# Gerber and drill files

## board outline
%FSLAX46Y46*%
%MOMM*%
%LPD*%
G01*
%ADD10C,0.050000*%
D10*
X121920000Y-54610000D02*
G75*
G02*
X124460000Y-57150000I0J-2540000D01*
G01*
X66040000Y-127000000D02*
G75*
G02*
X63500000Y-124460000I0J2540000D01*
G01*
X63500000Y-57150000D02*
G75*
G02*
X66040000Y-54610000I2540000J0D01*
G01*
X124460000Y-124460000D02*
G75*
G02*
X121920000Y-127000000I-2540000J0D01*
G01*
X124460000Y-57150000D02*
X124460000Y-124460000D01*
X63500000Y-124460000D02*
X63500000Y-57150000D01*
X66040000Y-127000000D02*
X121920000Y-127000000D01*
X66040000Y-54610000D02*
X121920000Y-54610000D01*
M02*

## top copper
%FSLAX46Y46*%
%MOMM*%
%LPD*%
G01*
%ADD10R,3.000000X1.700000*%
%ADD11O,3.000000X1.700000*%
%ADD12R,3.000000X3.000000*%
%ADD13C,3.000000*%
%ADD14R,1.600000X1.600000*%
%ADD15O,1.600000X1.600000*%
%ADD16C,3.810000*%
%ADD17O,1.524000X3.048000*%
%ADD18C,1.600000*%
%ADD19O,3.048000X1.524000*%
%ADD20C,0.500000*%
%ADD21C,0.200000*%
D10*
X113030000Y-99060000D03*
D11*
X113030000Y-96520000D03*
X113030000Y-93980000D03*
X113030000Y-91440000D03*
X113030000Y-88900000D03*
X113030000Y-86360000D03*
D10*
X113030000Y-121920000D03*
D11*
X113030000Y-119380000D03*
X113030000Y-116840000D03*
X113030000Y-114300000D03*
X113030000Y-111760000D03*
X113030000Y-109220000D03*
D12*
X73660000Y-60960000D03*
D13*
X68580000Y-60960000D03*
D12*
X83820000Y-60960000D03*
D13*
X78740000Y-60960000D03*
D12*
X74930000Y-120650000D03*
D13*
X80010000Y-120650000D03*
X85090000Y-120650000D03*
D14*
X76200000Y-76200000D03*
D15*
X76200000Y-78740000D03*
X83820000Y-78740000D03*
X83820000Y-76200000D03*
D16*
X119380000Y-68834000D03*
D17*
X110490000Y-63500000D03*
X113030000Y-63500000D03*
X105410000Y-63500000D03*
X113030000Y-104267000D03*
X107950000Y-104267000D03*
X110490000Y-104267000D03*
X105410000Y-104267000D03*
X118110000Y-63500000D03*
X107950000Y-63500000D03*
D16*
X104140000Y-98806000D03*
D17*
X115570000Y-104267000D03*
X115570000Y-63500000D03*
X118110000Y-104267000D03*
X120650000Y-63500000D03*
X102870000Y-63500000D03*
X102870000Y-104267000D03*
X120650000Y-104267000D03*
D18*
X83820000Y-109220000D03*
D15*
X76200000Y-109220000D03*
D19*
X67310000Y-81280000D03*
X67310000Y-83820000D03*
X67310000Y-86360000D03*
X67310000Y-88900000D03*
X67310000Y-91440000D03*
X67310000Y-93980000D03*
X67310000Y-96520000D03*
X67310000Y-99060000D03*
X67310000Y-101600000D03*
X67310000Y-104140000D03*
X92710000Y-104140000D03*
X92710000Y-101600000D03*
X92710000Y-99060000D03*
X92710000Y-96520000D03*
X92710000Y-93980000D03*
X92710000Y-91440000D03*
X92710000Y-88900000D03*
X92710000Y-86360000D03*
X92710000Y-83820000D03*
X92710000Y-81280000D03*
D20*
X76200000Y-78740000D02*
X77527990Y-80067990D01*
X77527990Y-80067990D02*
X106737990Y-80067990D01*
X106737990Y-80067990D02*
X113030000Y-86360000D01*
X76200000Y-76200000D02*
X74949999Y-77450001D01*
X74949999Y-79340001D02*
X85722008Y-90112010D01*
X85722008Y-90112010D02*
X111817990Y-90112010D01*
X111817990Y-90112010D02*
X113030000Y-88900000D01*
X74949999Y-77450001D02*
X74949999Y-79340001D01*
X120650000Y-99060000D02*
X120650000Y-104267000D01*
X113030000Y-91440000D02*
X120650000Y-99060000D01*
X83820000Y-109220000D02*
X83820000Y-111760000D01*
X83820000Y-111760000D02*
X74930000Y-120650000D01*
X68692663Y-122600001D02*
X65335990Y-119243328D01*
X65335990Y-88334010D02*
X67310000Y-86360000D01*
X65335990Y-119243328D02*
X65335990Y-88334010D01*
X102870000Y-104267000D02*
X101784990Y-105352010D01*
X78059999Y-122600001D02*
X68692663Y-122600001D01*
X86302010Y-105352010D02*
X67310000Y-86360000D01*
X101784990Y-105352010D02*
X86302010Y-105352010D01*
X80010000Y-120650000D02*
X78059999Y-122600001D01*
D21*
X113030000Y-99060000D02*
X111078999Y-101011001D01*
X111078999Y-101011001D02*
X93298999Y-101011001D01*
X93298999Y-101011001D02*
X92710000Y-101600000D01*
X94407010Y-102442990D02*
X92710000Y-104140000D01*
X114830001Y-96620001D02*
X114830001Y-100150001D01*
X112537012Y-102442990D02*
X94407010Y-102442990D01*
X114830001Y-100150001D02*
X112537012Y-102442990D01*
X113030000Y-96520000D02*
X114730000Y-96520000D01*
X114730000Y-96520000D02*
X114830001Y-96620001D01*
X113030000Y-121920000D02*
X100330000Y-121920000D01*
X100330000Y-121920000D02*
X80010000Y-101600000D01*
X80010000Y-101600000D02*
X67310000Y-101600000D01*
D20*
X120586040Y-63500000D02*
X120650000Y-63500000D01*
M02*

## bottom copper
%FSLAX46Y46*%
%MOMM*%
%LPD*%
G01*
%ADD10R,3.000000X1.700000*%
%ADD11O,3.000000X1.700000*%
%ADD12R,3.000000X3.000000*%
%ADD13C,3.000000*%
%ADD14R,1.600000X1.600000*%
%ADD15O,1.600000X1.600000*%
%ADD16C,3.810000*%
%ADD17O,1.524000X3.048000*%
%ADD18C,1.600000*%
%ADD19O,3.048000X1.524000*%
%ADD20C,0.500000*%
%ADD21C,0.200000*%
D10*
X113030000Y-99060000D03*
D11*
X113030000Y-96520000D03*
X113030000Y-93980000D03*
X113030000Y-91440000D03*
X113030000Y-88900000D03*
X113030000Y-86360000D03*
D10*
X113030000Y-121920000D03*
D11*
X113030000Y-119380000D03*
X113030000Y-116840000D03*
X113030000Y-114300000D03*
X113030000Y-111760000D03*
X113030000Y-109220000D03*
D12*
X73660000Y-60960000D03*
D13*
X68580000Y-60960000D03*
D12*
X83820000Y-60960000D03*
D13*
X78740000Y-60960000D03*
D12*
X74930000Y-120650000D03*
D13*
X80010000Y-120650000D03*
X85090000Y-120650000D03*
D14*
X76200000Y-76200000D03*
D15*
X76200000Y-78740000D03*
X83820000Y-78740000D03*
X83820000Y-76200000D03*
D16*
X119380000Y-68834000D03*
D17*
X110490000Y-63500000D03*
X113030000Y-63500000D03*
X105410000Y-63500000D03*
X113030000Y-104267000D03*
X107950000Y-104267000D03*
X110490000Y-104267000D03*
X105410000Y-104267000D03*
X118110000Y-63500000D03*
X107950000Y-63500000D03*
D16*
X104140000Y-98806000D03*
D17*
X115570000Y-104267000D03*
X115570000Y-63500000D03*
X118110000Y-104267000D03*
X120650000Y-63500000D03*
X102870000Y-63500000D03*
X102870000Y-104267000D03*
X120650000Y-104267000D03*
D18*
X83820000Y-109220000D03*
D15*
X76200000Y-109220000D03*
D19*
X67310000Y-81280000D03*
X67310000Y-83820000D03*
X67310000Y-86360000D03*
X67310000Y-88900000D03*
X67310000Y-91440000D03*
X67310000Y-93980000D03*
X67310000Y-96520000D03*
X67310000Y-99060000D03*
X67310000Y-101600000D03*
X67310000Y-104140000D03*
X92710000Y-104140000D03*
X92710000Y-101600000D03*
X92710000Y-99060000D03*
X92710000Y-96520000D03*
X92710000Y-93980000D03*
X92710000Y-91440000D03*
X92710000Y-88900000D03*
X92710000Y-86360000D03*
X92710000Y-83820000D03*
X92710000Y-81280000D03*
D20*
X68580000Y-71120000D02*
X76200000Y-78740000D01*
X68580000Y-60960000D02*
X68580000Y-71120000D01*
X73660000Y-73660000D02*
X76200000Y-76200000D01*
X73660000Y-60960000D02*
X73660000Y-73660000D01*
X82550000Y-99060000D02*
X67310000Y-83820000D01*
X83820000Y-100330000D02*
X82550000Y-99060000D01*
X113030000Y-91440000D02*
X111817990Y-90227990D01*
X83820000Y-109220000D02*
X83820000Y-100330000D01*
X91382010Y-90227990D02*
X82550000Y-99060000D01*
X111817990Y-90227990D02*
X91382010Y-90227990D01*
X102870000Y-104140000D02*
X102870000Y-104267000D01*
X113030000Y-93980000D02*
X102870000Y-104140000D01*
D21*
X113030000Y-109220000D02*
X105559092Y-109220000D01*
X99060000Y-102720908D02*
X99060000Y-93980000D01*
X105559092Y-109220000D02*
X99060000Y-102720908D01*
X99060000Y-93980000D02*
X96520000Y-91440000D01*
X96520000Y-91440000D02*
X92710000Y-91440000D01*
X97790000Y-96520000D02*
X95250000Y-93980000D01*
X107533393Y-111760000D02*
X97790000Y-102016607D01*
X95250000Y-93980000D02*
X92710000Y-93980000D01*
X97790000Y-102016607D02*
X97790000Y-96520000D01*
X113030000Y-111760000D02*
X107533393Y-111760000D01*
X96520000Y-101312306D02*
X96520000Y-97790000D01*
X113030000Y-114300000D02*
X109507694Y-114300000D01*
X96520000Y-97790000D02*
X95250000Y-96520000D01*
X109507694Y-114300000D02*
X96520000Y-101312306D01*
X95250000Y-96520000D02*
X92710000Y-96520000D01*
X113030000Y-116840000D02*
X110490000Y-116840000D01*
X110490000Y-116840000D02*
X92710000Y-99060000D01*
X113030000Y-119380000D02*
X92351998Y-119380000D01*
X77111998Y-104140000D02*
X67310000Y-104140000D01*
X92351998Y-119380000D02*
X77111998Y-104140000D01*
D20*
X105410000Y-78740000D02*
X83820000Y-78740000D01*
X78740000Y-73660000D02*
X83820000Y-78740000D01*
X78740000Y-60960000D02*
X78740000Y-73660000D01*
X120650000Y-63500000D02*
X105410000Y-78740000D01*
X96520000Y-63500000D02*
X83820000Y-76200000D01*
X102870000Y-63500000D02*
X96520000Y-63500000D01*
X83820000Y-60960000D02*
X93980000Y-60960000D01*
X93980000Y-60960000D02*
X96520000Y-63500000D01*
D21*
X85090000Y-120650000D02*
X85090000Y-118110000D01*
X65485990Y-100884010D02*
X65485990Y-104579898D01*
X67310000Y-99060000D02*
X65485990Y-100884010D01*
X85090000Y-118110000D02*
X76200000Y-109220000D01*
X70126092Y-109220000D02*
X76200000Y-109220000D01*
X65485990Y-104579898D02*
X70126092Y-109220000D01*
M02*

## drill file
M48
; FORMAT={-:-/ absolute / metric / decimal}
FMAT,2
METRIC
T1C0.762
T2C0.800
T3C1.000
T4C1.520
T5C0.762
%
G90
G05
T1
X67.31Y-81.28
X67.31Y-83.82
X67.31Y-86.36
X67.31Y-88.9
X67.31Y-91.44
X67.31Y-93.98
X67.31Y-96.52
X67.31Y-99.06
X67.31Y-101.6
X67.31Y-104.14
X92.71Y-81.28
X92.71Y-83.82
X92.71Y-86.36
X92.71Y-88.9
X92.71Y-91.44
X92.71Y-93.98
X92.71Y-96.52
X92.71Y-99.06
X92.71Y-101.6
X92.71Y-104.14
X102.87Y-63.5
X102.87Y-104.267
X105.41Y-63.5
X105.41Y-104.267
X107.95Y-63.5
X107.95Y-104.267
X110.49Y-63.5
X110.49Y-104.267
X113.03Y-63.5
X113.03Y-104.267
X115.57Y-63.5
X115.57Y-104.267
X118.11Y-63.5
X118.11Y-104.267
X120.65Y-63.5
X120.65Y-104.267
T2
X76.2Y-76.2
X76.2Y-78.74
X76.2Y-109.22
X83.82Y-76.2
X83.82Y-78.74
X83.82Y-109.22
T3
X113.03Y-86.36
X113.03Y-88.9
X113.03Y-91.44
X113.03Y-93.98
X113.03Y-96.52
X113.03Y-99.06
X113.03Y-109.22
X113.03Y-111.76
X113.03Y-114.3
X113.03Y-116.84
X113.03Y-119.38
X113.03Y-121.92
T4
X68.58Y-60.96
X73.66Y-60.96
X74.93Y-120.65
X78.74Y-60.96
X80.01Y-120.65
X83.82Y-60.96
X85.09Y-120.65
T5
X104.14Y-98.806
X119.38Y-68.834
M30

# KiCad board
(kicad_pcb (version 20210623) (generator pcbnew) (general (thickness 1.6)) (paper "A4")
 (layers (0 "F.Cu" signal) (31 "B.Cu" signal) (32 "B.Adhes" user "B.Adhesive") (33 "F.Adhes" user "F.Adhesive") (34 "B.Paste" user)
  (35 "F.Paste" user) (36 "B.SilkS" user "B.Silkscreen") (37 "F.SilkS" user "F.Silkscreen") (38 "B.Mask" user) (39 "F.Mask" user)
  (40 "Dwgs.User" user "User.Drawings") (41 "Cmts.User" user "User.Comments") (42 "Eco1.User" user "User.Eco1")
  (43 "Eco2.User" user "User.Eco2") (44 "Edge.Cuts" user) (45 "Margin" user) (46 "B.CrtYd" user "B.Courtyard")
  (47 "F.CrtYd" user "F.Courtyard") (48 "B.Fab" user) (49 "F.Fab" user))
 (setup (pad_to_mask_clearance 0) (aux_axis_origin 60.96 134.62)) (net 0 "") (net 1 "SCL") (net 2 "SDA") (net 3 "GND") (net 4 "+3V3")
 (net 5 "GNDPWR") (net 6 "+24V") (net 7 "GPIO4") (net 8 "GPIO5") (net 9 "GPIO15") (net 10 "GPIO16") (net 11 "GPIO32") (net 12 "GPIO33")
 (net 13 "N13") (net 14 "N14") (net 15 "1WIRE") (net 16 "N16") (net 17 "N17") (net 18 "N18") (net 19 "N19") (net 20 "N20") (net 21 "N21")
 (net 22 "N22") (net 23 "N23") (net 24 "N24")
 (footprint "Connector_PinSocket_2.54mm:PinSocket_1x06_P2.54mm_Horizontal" (layer "F.Cu") (at 113.03 99.06 180)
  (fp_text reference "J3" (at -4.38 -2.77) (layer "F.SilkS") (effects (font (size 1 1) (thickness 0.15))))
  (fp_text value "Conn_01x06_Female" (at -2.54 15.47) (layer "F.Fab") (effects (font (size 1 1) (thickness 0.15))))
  (pad "1" thru_hole rect locked (at 0 0 180) (size 3 1.7) (drill 1) (layers *.Cu *.Mask) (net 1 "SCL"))
  (pad "2" thru_hole oval locked (at 0 2.54 180) (size 3 1.7) (drill 1) (layers *.Cu *.Mask) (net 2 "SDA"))
  (pad "3" thru_hole oval locked (at 0 5.08 180) (size 3 1.7) (drill 1) (layers *.Cu *.Mask) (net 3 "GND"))
  (pad "4" thru_hole oval locked (at 0 7.62 180) (size 3 1.7) (drill 1) (layers *.Cu *.Mask) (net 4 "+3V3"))
  (pad "5" thru_hole oval locked (at 0 10.16 180) (size 3 1.7) (drill 1) (layers *.Cu *.Mask) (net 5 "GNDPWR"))
  (pad "6" thru_hole oval locked (at 0 12.7 180) (size 3 1.7) (drill 1) (layers *.Cu *.Mask) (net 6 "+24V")))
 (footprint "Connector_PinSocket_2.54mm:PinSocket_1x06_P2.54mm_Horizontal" (layer "F.Cu") (at 113.03 121.92 180)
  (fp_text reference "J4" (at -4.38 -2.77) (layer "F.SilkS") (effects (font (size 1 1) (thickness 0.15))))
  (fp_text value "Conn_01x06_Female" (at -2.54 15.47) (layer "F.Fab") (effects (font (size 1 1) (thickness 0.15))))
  (pad "1" thru_hole rect locked (at 0 0 180) (size 3 1.7) (drill 1) (layers *.Cu *.Mask) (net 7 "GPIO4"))
  (pad "2" thru_hole oval locked (at 0 2.54 180) (size 3 1.7) (drill 1) (layers *.Cu *.Mask) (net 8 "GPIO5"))
  (pad "3" thru_hole oval locked (at 0 5.08 180) (size 3 1.7) (drill 1) (layers *.Cu *.Mask) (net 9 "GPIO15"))
  (pad "4" thru_hole oval locked (at 0 7.62 180) (size 3 1.7) (drill 1) (layers *.Cu *.Mask) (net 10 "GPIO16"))
  (pad "5" thru_hole oval locked (at 0 10.16 180) (size 3 1.7) (drill 1) (layers *.Cu *.Mask) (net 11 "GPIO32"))
  (pad "6" thru_hole oval locked (at 0 12.7 180) (size 3 1.7) (drill 1) (layers *.Cu *.Mask) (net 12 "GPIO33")))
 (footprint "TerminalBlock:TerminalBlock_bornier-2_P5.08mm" (layer "F.Cu") (at 73.66 60.96 180)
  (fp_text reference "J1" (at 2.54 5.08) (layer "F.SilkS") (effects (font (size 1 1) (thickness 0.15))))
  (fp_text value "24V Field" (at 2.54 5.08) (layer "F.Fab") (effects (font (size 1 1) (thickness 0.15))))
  (pad "1" thru_hole rect locked (at 0 0 180) (size 3 3) (drill 1.52) (layers *.Cu *.Mask) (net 5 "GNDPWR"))
  (pad "2" thru_hole circle locked (at 5.08 0 180) (size 3 3) (drill 1.52) (layers *.Cu *.Mask) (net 6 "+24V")))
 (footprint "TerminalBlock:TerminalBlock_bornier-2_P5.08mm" (layer "F.Cu") (at 83.82 60.96 180)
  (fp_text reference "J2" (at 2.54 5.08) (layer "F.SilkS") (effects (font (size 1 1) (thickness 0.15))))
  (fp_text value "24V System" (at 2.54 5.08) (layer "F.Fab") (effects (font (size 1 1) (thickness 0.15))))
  (pad "1" thru_hole rect locked (at 0 0 180) (size 3 3) (drill 1.52) (layers *.Cu *.Mask) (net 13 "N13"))
  (pad "2" thru_hole circle locked (at 5.08 0 180) (size 3 3) (drill 1.52) (layers *.Cu *.Mask) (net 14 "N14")))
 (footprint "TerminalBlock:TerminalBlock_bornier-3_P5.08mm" (layer "F.Cu") (at 74.93 120.65)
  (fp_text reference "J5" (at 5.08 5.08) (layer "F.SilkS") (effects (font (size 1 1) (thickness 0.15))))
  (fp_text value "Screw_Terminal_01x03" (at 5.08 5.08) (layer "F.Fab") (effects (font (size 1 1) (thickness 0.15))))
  (pad "1" thru_hole rect locked (at 0 0) (size 3 3) (drill 1.52) (layers *.Cu *.Mask) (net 4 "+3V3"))
  (pad "2" thru_hole circle locked (at 5.08 0) (size 3 3) (drill 1.52) (layers *.Cu *.Mask) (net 3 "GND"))
  (pad "3" thru_hole circle locked (at 10.16 0) (size 3 3) (drill 1.52) (layers *.Cu *.Mask) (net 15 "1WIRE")))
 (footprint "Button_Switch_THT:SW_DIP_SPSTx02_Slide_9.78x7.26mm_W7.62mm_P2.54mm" (layer "F.Cu") (at 76.2 76.2)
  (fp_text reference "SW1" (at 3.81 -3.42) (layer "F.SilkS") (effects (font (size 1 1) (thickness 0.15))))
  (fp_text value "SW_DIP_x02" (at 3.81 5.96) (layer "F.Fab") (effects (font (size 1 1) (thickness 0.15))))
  (pad "1" thru_hole rect locked (at 0 0) (size 1.6 1.6) (drill 0.8) (layers *.Cu *.Mask) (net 5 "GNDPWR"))
  (pad "2" thru_hole oval locked (at 0 2.54) (size 1.6 1.6) (drill 0.8) (layers *.Cu *.Mask) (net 6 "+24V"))
  (pad "3" thru_hole oval locked (at 7.62 2.54) (size 1.6 1.6) (drill 0.8) (layers *.Cu *.Mask) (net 14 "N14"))
  (pad "4" thru_hole oval locked (at 7.62 0) (size 1.6 1.6) (drill 0.8) (layers *.Cu *.Mask) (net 13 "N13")))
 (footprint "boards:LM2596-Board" (layer "F.Cu") (at 111.76 83.82 -90)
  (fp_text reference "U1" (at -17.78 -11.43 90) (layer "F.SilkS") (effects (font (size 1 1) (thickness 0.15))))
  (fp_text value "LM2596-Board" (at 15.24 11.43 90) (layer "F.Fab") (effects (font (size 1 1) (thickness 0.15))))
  (pad "" np_thru_hole circle locked (at -14.986 -7.62 270) (size 3.81 3.81) (drill 0.762) (layers *.Cu *.Mask))
  (pad "" thru_hole oval locked (at -20.32 1.27 270) (size 3.048 1.524) (drill 0.762) (layers *.Cu *.Mask))
  (pad "" thru_hole oval locked (at -20.32 -1.27 270) (size 3.048 1.524) (drill 0.762) (layers *.Cu *.Mask))
  (pad "" thru_hole oval locked (at -20.32 6.35 270) (size 3.048 1.524) (drill 0.762) (layers *.Cu *.Mask))
  (pad "" thru_hole oval locked (at 20.447 -1.27 270) (size 3.048 1.524) (drill 0.762) (layers *.Cu *.Mask))
  (pad "" thru_hole oval locked (at 20.447 3.81 270) (size 3.048 1.524) (drill 0.762) (layers *.Cu *.Mask))
  (pad "" thru_hole oval locked (at 20.447 1.27 270) (size 3.048 1.524) (drill 0.762) (layers *.Cu *.Mask))
  (pad "" thru_hole oval locked (at 20.447 6.35 270) (size 3.048 1.524) (drill 0.762) (layers *.Cu *.Mask))
  (pad "" thru_hole oval locked (at -20.32 -6.35 270) (size 3.048 1.524) (drill 0.762) (layers *.Cu *.Mask))
  (pad "" thru_hole oval locked (at -20.32 3.81 270) (size 3.048 1.524) (drill 0.762) (layers *.Cu *.Mask))
  (pad "" np_thru_hole circle locked (at 14.986 7.62 270) (size 3.81 3.81) (drill 0.762) (layers *.Cu *.Mask))
  (pad "" thru_hole oval locked (at 20.447 -3.81 270) (size 3.048 1.524) (drill 0.762) (layers *.Cu *.Mask))
  (pad "" thru_hole oval locked (at -20.32 -3.81 270) (size 3.048 1.524) (drill 0.762) (layers *.Cu *.Mask))
  (pad "" thru_hole oval locked (at 20.447 -6.35 270) (size 3.048 1.524) (drill 0.762) (layers *.Cu *.Mask))
  (pad "1" thru_hole oval locked (at -20.32 -8.89 270) (size 3.048 1.524) (drill 0.762) (layers *.Cu *.Mask) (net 14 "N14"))
  (pad "2" thru_hole oval locked (at -20.32 8.89 270) (size 3.048 1.524) (drill 0.762) (layers *.Cu *.Mask) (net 13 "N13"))
  (pad "3" thru_hole oval locked (at 20.447 8.89 270) (size 3.048 1.524) (drill 0.762) (layers *.Cu *.Mask) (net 3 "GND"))
  (pad "4" thru_hole oval locked (at 20.447 -8.89 270) (size 3.048 1.524) (drill 0.762) (layers *.Cu *.Mask) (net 4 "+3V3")))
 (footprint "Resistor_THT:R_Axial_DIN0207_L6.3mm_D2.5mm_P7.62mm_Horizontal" (layer "F.Cu") (at 83.82 109.22 180)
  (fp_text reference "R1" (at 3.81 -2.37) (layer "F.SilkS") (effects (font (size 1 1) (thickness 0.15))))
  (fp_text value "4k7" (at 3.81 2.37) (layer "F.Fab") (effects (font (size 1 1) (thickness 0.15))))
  (pad "1" thru_hole circle locked (at 0 0 180) (size 1.6 1.6) (drill 0.8) (layers *.Cu *.Mask) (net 4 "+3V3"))
  (pad "2" thru_hole oval locked (at 7.62 0 180) (size 1.6 1.6) (drill 0.8) (layers *.Cu *.Mask) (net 15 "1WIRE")))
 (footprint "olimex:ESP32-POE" (layer "F.Cu") (at 80.01 90.17)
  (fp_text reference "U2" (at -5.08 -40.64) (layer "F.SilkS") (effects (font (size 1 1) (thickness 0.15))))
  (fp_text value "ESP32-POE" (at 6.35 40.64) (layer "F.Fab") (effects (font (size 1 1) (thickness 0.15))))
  (pad "1" thru_hole oval locked (at -12.7 -8.89) (size 3.048 1.524) (drill 0.762) (layers *.Cu *.Mask) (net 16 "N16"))
  (pad "2" thru_hole oval locked (at -12.7 -6.35) (size 3.048 1.524) (drill 0.762) (layers *.Cu *.Mask) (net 4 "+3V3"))
  (pad "3" thru_hole oval locked (at -12.7 -3.81) (size 3.048 1.524) (drill 0.762) (layers *.Cu *.Mask) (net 3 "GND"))
  (pad "4" thru_hole oval locked (at -12.7 -1.27) (size 3.048 1.524) (drill 0.762) (layers *.Cu *.Mask) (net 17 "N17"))
  (pad "5" thru_hole oval locked (at -12.7 1.27) (size 3.048 1.524) (drill 0.762) (layers *.Cu *.Mask) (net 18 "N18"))
  (pad "6" thru_hole oval locked (at -12.7 3.81) (size 3.048 1.524) (drill 0.762) (layers *.Cu *.Mask) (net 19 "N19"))
  (pad "7" thru_hole oval locked (at -12.7 6.35) (size 3.048 1.524) (drill 0.762) (layers *.Cu *.Mask) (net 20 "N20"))
  (pad "8" thru_hole oval locked (at -12.7 8.89) (size 3.048 1.524) (drill 0.762) (layers *.Cu *.Mask) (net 15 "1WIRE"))
  (pad "9" thru_hole oval locked (at -12.7 11.43) (size 3.048 1.524) (drill 0.762) (layers *.Cu *.Mask) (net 7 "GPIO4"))
  (pad "10" thru_hole oval locked (at -12.7 13.97) (size 3.048 1.524) (drill 0.762) (layers *.Cu *.Mask) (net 8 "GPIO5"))
  (pad "11" thru_hole oval locked (at 12.7 13.97) (size 3.048 1.524) (drill 0.762) (layers *.Cu *.Mask) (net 2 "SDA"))
  (pad "12" thru_hole oval locked (at 12.7 11.43) (size 3.048 1.524) (drill 0.762) (layers *.Cu *.Mask) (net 1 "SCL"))
  (pad "13" thru_hole oval locked (at 12.7 8.89) (size 3.048 1.524) (drill 0.762) (layers *.Cu *.Mask) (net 9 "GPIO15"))
  (pad "14" thru_hole oval locked (at 12.7 6.35) (size 3.048 1.524) (drill 0.762) (layers *.Cu *.Mask) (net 10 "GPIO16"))
  (pad "15" thru_hole oval locked (at 12.7 3.81) (size 3.048 1.524) (drill 0.762) (layers *.Cu *.Mask) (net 11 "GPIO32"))
  (pad "16" thru_hole oval locked (at 12.7 1.27) (size 3.048 1.524) (drill 0.762) (layers *.Cu *.Mask) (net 12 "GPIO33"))
  (pad "17" thru_hole oval locked (at 12.7 -1.27) (size 3.048 1.524) (drill 0.762) (layers *.Cu *.Mask) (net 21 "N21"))
  (pad "18" thru_hole oval locked (at 12.7 -3.81) (size 3.048 1.524) (drill 0.762) (layers *.Cu *.Mask) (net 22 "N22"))
  (pad "19" thru_hole oval locked (at 12.7 -6.35) (size 3.048 1.524) (drill 0.762) (layers *.Cu *.Mask) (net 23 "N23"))
  (pad "20" thru_hole oval locked (at 12.7 -8.89) (size 3.048 1.524) (drill 0.762) (layers *.Cu *.Mask) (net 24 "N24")))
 (gr_arc (start 121.92 57.15) (end 124.46 57.15) (angle -90) (layer "Edge.Cuts") (width 0.05))
 (gr_arc (start 66.04 124.46) (end 63.5 124.46) (angle -90) (layer "Edge.Cuts") (width 0.05))
 (gr_arc (start 66.04 57.15) (end 66.04 54.61) (angle -90) (layer "Edge.Cuts") (width 0.05))
 (gr_arc (start 121.92 124.46) (end 121.92 127) (angle -90) (layer "Edge.Cuts") (width 0.05))
 (gr_line (start 124.46 57.15) (end 124.46 124.46) (layer "Edge.Cuts") (width 0.05))
 (gr_line (start 63.5 124.46) (end 63.5 57.15) (layer "Edge.Cuts") (width 0.05))
 (gr_line (start 66.04 127) (end 121.92 127) (layer "Edge.Cuts") (width 0.05))
 (gr_line (start 66.04 54.61) (end 121.92 54.61) (layer "Edge.Cuts") (width 0.05))
 (segment (start 76.2 78.74) (end 77.52799 80.06799) (width 0.5) (layer "F.Cu") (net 6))
 (segment (start 77.52799 80.06799) (end 106.73799 80.06799) (width 0.5) (layer "F.Cu") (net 6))
 (segment (start 106.73799 80.06799) (end 113.03 86.36) (width 0.5) (layer "F.Cu") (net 6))
 (segment (start 68.58 71.12) (end 76.2 78.74) (width 0.5) (layer "B.Cu") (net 6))
 (segment (start 68.58 60.96) (end 68.58 71.12) (width 0.5) (layer "B.Cu") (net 6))
 (segment (start 76.2 76.2) (end 74.949999 77.450001) (width 0.5) (layer "F.Cu") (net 5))
 (segment (start 74.949999 79.340001) (end 85.722008 90.11201) (width 0.5) (layer "F.Cu") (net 5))
 (segment (start 85.722008 90.11201) (end 111.81799 90.11201) (width 0.5) (layer "F.Cu") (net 5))
 (segment (start 111.81799 90.11201) (end 113.03 88.9) (width 0.5) (layer "F.Cu") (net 5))
 (segment (start 74.949999 77.450001) (end 74.949999 79.340001) (width 0.5) (layer "F.Cu") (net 5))
 (segment (start 73.66 73.66) (end 76.2 76.2) (width 0.5) (layer "B.Cu") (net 5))
 (segment (start 73.66 60.96) (end 73.66 73.66) (width 0.5) (layer "B.Cu") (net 5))
 (segment (start 120.65 99.06) (end 120.65 104.267) (width 0.5) (layer "F.Cu") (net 4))
 (segment (start 113.03 91.44) (end 120.65 99.06) (width 0.5) (layer "F.Cu") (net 4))
 (segment (start 83.82 109.22) (end 83.82 111.76) (width 0.5) (layer "F.Cu") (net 4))
 (segment (start 83.82 111.76) (end 74.93 120.65) (width 0.5) (layer "F.Cu") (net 4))
 (segment (start 82.55 99.06) (end 67.31 83.82) (width 0.5) (layer "B.Cu") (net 4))
 (segment (start 83.82 100.33) (end 82.55 99.06) (width 0.5) (layer "B.Cu") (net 4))
 (segment (start 113.03 91.44) (end 111.81799 90.22799) (width 0.5) (layer "B.Cu") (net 4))
 (segment (start 83.82 109.22) (end 83.82 100.33) (width 0.5) (layer "B.Cu") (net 4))
 (segment (start 91.38201 90.22799) (end 82.55 99.06) (width 0.5) (layer "B.Cu") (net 4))
 (segment (start 111.81799 90.22799) (end 91.38201 90.22799) (width 0.5) (layer "B.Cu") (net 4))
 (segment (start 68.692663 122.600001) (end 65.33599 119.243328) (width 0.5) (layer "F.Cu") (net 3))
 (segment (start 65.33599 88.33401) (end 67.31 86.36) (width 0.5) (layer "F.Cu") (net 3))
 (segment (start 65.33599 119.243328) (end 65.33599 88.33401) (width 0.5) (layer "F.Cu") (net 3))
 (segment (start 102.87 104.267) (end 101.78499 105.35201) (width 0.5) (layer "F.Cu") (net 3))
 (segment (start 78.059999 122.600001) (end 68.692663 122.600001) (width 0.5) (layer "F.Cu") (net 3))
 (segment (start 86.30201 105.35201) (end 67.31 86.36) (width 0.5) (layer "F.Cu") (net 3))
 (segment (start 101.78499 105.35201) (end 86.30201 105.35201) (width 0.5) (layer "F.Cu") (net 3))
 (segment (start 80.01 120.65) (end 78.059999 122.600001) (width 0.5) (layer "F.Cu") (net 3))
 (segment (start 102.87 104.14) (end 102.87 104.267) (width 0.5) (layer "B.Cu") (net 3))
 (segment (start 113.03 93.98) (end 102.87 104.14) (width 0.5) (layer "B.Cu") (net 3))
 (segment (start 113.03 99.06) (end 111.078999 101.011001) (width 0.2) (layer "F.Cu") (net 1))
 (segment (start 111.078999 101.011001) (end 93.298999 101.011001) (width 0.2) (layer "F.Cu") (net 1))
 (segment (start 93.298999 101.011001) (end 92.71 101.6) (width 0.2) (layer "F.Cu") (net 1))
 (segment (start 94.40701 102.44299) (end 92.71 104.14) (width 0.2) (layer "F.Cu") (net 2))
 (segment (start 114.830001 96.620001) (end 114.830001 100.150001) (width 0.2) (layer "F.Cu") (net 2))
 (segment (start 112.537012 102.44299) (end 94.40701 102.44299) (width 0.2) (layer "F.Cu") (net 2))
 (segment (start 114.830001 100.150001) (end 112.537012 102.44299) (width 0.2) (layer "F.Cu") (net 2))
 (segment (start 113.03 96.52) (end 114.73 96.52) (width 0.2) (layer "F.Cu") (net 2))
 (segment (start 114.73 96.52) (end 114.830001 96.620001) (width 0.2) (layer "F.Cu") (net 2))
 (segment (start 113.03 109.22) (end 105.559092 109.22) (width 0.2) (layer "B.Cu") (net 12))
 (segment (start 99.06 102.720908) (end 99.06 93.98) (width 0.2) (layer "B.Cu") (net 12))
 (segment (start 105.559092 109.22) (end 99.06 102.720908) (width 0.2) (layer "B.Cu") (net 12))
 (segment (start 99.06 93.98) (end 96.52 91.44) (width 0.2) (layer "B.Cu") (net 12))
 (segment (start 96.52 91.44) (end 92.71 91.44) (width 0.2) (layer "B.Cu") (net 12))
 (segment (start 97.79 96.52) (end 95.25 93.98) (width 0.2) (layer "B.Cu") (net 11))
 (segment (start 107.533393 111.76) (end 97.79 102.016607) (width 0.2) (layer "B.Cu") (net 11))
 (segment (start 95.25 93.98) (end 92.71 93.98) (width 0.2) (layer "B.Cu") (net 11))
 (segment (start 97.79 102.016607) (end 97.79 96.52) (width 0.2) (layer "B.Cu") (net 11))
 (segment (start 113.03 111.76) (end 107.533393 111.76) (width 0.2) (layer "B.Cu") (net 11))
 (segment (start 96.52 101.312306) (end 96.52 97.79) (width 0.2) (layer "B.Cu") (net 10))
 (segment (start 113.03 114.3) (end 109.507694 114.3) (width 0.2) (layer "B.Cu") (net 10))
 (segment (start 96.52 97.79) (end 95.25 96.52) (width 0.2) (layer "B.Cu") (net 10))
 (segment (start 109.507694 114.3) (end 96.52 101.312306) (width 0.2) (layer "B.Cu") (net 10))
 (segment (start 95.25 96.52) (end 92.71 96.52) (width 0.2) (layer "B.Cu") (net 10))
 (segment (start 113.03 116.84) (end 110.49 116.84) (width 0.2) (layer "B.Cu") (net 9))
 (segment (start 110.49 116.84) (end 92.71 99.06) (width 0.2) (layer "B.Cu") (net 9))
 (segment (start 113.03 119.38) (end 92.351998 119.38) (width 0.2) (layer "B.Cu") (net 8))
 (segment (start 77.111998 104.14) (end 67.31 104.14) (width 0.2) (layer "B.Cu") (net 8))
 (segment (start 92.351998 119.38) (end 77.111998 104.14) (width 0.2) (layer "B.Cu") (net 8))
 (segment (start 113.03 121.92) (end 100.33 121.92) (width 0.2) (layer "F.Cu") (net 7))
 (segment (start 100.33 121.92) (end 80.01 101.6) (width 0.2) (layer "F.Cu") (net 7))
 (segment (start 80.01 101.6) (end 67.31 101.6) (width 0.2) (layer "F.Cu") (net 7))
 (segment (start 120.58604 63.5) (end 120.65 63.5) (width 0.5) (layer "F.Cu") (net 14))
 (segment (start 105.41 78.74) (end 83.82 78.74) (width 0.5) (layer "B.Cu") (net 14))
 (segment (start 78.74 73.66) (end 83.82 78.74) (width 0.5) (layer "B.Cu") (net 14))
 (segment (start 78.74 60.96) (end 78.74 73.66) (width 0.5) (layer "B.Cu") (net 14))
 (segment (start 120.65 63.5) (end 105.41 78.74) (width 0.5) (layer "B.Cu") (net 14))
 (segment (start 96.52 63.5) (end 83.82 76.2) (width 0.5) (layer "B.Cu") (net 13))
 (segment (start 102.87 63.5) (end 96.52 63.5) (width 0.5) (layer "B.Cu") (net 13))
 (segment (start 83.82 60.96) (end 93.98 60.96) (width 0.5) (layer "B.Cu") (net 13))
 (segment (start 93.98 60.96) (end 96.52 63.5) (width 0.5) (layer "B.Cu") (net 13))
 (segment (start 85.09 120.65) (end 85.09 118.11) (width 0.2) (layer "B.Cu") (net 15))
 (segment (start 65.48599 100.88401) (end 65.48599 104.579898) (width 0.2) (layer "B.Cu") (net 15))
 (segment (start 67.31 99.06) (end 65.48599 100.88401) (width 0.2) (layer "B.Cu") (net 15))
 (segment (start 85.09 118.11) (end 76.2 109.22) (width 0.2) (layer "B.Cu") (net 15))
 (segment (start 70.126092 109.22) (end 76.2 109.22) (width 0.2) (layer "B.Cu") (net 15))
 (segment (start 65.48599 104.579898) (end 70.126092 109.22) (width 0.2) (layer "B.Cu") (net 15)))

